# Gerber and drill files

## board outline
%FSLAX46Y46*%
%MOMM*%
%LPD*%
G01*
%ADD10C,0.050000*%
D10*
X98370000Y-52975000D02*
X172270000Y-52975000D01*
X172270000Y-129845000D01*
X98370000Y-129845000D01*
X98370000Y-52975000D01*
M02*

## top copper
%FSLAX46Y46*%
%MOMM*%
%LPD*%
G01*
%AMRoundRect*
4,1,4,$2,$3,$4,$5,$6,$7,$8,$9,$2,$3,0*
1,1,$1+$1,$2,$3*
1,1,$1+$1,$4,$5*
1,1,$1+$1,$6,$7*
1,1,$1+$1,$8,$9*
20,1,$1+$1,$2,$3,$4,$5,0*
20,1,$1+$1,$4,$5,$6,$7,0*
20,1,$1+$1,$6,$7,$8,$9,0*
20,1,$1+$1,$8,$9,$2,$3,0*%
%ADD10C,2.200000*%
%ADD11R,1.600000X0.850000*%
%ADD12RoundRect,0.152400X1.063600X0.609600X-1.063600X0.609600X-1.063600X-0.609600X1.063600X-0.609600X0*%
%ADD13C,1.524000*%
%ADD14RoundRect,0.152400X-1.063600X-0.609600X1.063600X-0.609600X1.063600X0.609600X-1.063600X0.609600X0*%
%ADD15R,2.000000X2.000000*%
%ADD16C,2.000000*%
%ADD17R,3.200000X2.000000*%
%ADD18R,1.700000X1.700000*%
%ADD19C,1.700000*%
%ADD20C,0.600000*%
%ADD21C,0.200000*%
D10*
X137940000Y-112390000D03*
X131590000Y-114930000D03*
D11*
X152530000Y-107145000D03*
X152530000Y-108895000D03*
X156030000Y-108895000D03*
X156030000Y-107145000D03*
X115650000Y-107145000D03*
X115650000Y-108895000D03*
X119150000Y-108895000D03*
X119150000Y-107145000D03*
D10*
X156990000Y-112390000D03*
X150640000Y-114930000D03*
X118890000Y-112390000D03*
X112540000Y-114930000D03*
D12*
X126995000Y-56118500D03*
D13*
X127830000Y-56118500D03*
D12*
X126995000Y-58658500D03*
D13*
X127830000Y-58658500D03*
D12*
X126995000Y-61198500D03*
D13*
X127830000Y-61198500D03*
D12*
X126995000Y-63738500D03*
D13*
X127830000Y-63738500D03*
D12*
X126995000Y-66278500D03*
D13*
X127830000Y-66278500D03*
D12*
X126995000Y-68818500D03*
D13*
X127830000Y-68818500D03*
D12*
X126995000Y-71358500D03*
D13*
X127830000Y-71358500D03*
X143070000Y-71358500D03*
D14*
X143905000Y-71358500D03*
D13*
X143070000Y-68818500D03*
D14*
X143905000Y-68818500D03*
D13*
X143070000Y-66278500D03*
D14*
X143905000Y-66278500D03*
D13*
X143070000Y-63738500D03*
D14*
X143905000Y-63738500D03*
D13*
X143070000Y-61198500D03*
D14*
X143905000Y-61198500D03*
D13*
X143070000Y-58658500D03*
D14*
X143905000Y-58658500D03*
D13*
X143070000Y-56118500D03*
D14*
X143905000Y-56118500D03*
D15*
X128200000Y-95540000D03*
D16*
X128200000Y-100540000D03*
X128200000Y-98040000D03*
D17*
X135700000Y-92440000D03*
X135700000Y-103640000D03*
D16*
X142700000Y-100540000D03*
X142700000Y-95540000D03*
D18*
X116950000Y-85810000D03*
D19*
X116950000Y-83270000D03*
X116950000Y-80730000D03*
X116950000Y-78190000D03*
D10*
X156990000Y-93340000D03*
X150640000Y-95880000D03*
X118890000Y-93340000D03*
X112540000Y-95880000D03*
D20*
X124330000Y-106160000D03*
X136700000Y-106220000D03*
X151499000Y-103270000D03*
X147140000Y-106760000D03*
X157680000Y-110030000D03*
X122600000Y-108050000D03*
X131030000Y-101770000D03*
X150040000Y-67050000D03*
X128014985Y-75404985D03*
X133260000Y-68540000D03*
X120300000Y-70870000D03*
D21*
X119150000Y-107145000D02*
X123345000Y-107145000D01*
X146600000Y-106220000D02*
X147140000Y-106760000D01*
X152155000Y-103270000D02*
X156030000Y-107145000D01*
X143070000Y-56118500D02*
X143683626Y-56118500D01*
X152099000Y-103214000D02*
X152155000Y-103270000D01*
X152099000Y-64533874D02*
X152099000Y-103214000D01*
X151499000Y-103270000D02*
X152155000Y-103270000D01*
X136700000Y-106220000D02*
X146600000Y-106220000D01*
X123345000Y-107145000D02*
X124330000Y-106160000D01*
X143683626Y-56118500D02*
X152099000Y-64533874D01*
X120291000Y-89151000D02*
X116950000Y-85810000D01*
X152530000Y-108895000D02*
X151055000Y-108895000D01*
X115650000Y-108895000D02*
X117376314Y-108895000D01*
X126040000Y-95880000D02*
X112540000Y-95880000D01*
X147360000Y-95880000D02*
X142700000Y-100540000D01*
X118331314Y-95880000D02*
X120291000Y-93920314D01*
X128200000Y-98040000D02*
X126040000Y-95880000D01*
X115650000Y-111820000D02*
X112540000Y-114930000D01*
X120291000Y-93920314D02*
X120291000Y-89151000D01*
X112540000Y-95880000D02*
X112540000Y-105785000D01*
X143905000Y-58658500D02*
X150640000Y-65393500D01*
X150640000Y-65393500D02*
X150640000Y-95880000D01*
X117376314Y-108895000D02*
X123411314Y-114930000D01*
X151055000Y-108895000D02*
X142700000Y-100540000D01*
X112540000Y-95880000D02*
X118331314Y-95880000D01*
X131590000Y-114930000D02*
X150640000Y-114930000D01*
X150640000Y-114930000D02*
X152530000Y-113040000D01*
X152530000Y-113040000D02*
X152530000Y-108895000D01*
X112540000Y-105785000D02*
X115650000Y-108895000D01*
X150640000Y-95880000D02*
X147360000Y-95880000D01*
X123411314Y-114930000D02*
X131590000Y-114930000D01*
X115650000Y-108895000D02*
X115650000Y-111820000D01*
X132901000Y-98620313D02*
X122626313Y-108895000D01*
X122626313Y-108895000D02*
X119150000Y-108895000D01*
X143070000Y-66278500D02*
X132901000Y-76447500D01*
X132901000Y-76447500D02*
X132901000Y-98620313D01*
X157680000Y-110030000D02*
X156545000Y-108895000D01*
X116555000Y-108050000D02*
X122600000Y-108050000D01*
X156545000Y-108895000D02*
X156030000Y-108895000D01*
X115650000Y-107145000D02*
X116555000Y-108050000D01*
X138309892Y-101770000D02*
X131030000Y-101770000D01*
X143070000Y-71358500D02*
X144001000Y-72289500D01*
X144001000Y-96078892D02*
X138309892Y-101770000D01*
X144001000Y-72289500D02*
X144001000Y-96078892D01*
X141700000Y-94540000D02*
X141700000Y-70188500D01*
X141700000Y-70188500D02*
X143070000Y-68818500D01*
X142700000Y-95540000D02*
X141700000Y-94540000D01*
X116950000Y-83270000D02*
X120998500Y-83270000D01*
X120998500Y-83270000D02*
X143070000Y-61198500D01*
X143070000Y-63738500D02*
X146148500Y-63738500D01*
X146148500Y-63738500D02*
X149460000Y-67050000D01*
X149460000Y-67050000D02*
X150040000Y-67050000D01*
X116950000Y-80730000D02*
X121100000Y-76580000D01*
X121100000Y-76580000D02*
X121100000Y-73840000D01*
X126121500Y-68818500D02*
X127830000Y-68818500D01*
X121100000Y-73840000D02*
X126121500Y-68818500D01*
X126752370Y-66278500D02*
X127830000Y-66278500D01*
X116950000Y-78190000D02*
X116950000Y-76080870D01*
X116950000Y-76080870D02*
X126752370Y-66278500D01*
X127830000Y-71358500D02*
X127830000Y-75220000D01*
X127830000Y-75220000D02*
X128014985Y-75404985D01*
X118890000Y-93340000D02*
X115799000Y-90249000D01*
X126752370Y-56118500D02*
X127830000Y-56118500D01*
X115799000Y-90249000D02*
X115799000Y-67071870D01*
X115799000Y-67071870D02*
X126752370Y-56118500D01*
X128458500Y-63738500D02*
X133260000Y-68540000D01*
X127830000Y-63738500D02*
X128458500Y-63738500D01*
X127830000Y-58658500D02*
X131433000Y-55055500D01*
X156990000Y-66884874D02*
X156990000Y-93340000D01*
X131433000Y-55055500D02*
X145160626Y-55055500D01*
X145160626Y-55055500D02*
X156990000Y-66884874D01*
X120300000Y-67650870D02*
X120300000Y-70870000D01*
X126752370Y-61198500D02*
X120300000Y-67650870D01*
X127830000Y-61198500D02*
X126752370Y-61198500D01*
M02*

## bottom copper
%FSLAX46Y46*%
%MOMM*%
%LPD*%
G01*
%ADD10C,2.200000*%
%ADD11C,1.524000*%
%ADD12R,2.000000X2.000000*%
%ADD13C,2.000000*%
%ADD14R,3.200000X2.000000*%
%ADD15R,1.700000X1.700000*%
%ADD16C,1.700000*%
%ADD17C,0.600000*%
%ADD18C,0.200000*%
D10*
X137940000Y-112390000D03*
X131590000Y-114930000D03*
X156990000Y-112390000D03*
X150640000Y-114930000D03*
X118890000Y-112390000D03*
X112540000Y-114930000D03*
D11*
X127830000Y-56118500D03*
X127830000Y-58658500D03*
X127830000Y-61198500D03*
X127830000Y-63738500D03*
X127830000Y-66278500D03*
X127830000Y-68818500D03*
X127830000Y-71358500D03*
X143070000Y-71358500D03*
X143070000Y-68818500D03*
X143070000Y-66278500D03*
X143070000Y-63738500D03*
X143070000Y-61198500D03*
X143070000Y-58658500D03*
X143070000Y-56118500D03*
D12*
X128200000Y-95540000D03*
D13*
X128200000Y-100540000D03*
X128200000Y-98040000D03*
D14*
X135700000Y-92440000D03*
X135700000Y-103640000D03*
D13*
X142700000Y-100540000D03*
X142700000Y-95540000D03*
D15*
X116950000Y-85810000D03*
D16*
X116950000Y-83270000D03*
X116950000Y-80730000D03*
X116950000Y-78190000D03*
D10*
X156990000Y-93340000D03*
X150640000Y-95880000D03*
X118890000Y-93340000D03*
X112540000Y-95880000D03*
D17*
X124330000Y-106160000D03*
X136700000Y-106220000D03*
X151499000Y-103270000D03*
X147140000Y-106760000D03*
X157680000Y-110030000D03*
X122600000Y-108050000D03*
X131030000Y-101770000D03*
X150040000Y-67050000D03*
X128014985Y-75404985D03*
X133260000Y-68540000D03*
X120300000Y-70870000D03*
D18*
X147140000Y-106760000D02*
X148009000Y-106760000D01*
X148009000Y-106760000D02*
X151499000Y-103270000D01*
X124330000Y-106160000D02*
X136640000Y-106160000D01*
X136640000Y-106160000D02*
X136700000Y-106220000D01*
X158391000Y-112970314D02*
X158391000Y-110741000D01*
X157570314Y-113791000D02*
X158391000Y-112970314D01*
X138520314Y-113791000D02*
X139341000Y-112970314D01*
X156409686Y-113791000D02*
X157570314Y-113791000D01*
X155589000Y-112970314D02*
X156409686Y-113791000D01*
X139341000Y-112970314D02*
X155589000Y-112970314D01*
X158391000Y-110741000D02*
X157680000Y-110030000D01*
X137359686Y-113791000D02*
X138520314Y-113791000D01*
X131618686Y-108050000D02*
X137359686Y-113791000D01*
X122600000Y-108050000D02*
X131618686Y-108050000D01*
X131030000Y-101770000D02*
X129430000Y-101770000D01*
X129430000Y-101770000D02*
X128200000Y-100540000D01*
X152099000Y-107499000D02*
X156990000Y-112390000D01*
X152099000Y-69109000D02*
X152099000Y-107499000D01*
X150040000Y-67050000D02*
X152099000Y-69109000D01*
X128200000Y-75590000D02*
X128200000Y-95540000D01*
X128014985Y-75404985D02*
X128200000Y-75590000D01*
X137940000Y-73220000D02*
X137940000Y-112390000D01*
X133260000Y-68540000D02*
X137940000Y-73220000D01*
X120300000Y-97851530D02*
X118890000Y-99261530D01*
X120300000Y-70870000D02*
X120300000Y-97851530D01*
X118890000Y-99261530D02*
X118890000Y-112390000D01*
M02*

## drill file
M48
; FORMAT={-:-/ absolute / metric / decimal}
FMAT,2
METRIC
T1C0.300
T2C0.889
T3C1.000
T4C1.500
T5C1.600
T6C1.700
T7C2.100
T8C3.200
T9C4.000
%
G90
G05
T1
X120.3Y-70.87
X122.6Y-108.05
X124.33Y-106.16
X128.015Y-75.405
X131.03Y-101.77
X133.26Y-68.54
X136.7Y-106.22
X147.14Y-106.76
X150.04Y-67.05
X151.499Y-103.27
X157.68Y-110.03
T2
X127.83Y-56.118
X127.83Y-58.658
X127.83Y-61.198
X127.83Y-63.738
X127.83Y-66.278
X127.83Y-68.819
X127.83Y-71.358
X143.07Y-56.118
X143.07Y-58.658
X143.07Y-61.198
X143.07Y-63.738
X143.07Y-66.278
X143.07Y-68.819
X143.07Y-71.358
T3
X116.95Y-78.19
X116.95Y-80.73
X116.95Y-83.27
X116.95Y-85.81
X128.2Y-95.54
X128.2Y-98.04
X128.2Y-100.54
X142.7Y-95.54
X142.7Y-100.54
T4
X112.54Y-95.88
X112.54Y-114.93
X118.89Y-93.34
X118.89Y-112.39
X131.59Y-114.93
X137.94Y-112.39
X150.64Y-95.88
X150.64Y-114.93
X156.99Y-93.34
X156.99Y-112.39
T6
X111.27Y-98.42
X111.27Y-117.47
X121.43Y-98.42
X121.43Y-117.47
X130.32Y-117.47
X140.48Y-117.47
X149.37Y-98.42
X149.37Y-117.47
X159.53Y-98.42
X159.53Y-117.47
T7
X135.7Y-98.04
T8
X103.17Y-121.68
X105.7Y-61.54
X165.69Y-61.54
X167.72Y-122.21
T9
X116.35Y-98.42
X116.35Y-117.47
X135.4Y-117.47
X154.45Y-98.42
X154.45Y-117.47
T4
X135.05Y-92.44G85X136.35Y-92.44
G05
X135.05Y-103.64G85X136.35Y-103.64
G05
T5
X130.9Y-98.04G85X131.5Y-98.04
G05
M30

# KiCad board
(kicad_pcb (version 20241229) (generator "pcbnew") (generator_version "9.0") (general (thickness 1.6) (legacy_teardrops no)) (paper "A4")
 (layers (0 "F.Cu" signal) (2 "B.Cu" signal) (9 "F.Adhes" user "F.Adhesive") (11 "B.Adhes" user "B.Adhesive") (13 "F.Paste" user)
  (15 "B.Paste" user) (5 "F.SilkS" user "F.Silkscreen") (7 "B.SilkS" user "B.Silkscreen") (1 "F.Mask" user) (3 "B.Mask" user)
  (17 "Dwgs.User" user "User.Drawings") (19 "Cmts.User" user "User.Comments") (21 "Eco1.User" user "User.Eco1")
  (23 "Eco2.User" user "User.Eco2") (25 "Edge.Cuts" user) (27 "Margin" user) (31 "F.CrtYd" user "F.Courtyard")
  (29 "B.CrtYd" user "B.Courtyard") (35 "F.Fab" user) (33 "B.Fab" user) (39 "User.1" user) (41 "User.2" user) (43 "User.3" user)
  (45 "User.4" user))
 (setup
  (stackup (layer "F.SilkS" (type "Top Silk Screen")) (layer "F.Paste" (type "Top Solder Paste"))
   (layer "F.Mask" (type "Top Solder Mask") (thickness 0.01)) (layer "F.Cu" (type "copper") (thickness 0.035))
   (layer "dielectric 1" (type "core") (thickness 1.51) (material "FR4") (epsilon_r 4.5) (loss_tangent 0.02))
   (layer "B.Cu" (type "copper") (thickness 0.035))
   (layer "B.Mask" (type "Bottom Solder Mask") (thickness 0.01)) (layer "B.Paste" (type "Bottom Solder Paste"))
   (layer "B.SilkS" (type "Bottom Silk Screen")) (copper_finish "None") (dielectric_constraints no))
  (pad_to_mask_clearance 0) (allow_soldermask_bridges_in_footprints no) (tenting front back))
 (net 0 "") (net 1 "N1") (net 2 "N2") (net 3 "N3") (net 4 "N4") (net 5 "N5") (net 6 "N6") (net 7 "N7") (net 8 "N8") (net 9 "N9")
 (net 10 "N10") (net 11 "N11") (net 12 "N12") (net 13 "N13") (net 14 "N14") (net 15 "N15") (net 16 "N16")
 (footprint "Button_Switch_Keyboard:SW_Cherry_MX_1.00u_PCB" (layer "F.Cu") (at 137.94 112.39)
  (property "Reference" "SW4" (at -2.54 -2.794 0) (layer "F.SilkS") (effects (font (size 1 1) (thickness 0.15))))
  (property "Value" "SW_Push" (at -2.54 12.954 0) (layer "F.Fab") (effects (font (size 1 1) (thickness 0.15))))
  (pad "" np_thru_hole circle (at -7.62 5.08) (size 1.7 1.7) (drill 1.7) (layers "*.Cu" "*.Mask"))
  (pad "" np_thru_hole circle (at -2.54 5.08) (size 4 4) (drill 4) (layers "*.Cu" "*.Mask"))
  (pad "" np_thru_hole circle (at 2.54 5.08) (size 1.7 1.7) (drill 1.7) (layers "*.Cu" "*.Mask"))
  (pad "1" thru_hole circle (at 0 0) (size 2.2 2.2) (drill 1.5) (layers "*.Cu" "*.Mask") (remove_unused_layers no) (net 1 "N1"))
  (pad "2" thru_hole circle (at -6.35 2.54) (size 2.2 2.2) (drill 1.5) (layers "*.Cu" "*.Mask") (remove_unused_layers no) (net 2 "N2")))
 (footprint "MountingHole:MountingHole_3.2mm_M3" (layer "F.Cu") (at 105.7 61.54 -90)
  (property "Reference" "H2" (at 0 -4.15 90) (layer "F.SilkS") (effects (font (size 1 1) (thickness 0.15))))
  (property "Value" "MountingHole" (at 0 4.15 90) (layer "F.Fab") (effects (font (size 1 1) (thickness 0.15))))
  (pad "" np_thru_hole circle (at 0 0 270) (size 3.2 3.2) (drill 3.2) (layers "*.Cu" "*.Mask")))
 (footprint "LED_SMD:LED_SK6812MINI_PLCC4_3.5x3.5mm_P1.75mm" (layer "F.Cu") (at 154.28 108.02)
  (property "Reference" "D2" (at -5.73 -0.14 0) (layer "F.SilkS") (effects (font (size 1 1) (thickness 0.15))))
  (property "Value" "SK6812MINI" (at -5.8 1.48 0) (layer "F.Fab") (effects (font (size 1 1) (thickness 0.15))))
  (pad "1" smd rect (at -1.75 -0.875) (size 1.6 0.85) (layers "F.Cu" "F.Mask" "F.Paste") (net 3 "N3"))
  (pad "2" smd rect (at -1.75 0.875) (size 1.6 0.85) (layers "F.Cu" "F.Mask" "F.Paste") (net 2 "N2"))
  (pad "3" smd rect (at 1.75 0.875) (size 1.6 0.85) (layers "F.Cu" "F.Mask" "F.Paste") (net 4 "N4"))
  (pad "4" smd rect (at 1.75 -0.875) (size 1.6 0.85) (layers "F.Cu" "F.Mask" "F.Paste") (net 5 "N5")))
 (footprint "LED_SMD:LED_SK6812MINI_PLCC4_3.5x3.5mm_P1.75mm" (layer "F.Cu") (at 117.4 108.02)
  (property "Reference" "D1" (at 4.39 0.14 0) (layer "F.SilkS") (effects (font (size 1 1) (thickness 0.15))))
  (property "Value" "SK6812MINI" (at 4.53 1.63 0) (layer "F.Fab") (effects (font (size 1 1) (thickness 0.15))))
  (pad "1" smd rect (at -1.75 -0.875) (size 1.6 0.85) (layers "F.Cu" "F.Mask" "F.Paste") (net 4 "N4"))
  (pad "2" smd rect (at -1.75 0.875) (size 1.6 0.85) (layers "F.Cu" "F.Mask" "F.Paste") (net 2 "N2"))
  (pad "3" smd rect (at 1.75 0.875) (size 1.6 0.85) (layers "F.Cu" "F.Mask" "F.Paste") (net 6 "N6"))
  (pad "4" smd rect (at 1.75 -0.875) (size 1.6 0.85) (layers "F.Cu" "F.Mask" "F.Paste") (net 5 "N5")))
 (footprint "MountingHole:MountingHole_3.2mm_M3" (layer "F.Cu") (at 165.69 61.54 90)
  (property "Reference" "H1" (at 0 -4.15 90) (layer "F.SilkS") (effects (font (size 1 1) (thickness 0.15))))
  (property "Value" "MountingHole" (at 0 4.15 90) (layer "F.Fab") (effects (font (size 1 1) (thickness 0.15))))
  (pad "" np_thru_hole circle (at 0 0 90) (size 3.2 3.2) (drill 3.2) (layers "*.Cu" "*.Mask")))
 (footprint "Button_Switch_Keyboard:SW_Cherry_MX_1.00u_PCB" (layer "F.Cu") (at 156.99 112.39)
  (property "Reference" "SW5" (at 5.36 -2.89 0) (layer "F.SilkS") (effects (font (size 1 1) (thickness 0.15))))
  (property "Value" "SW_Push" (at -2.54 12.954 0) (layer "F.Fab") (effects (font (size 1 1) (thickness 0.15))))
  (pad "" np_thru_hole circle (at -7.62 5.08) (size 1.7 1.7) (drill 1.7) (layers "*.Cu" "*.Mask"))
  (pad "" np_thru_hole circle (at -2.54 5.08) (size 4 4) (drill 4) (layers "*.Cu" "*.Mask"))
  (pad "" np_thru_hole circle (at 2.54 5.08) (size 1.7 1.7) (drill 1.7) (layers "*.Cu" "*.Mask"))
  (pad "1" thru_hole circle (at 0 0) (size 2.2 2.2) (drill 1.5) (layers "*.Cu" "*.Mask") (remove_unused_layers no) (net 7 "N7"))
  (pad "2" thru_hole circle (at -6.35 2.54) (size 2.2 2.2) (drill 1.5) (layers "*.Cu" "*.Mask") (remove_unused_layers no) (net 2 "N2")))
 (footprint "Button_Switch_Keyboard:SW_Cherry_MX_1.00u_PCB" (layer "F.Cu") (at 118.89 112.39)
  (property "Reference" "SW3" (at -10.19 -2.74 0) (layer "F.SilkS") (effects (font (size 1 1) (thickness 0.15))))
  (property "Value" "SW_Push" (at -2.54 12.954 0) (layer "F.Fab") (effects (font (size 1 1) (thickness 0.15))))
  (pad "" np_thru_hole circle (at -7.62 5.08) (size 1.7 1.7) (drill 1.7) (layers "*.Cu" "*.Mask"))
  (pad "" np_thru_hole circle (at -2.54 5.08) (size 4 4) (drill 4) (layers "*.Cu" "*.Mask"))
  (pad "" np_thru_hole circle (at 2.54 5.08) (size 1.7 1.7) (drill 1.7) (layers "*.Cu" "*.Mask"))
  (pad "1" thru_hole circle (at 0 0) (size 2.2 2.2) (drill 1.5) (layers "*.Cu" "*.Mask") (remove_unused_layers no) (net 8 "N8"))
  (pad "2" thru_hole circle (at -6.35 2.54) (size 2.2 2.2) (drill 1.5) (layers "*.Cu" "*.Mask") (remove_unused_layers no) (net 2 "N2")))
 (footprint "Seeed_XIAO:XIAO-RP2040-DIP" (layer "F.Cu") (at 135.45 63.7385)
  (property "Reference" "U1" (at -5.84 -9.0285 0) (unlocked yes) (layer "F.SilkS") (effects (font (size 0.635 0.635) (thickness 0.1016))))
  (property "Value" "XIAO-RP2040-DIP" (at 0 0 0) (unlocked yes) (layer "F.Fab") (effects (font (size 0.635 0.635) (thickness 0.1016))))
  (pad "1" smd roundrect (at -8.455 -7.62 180) (size 2.432 1.524) (layers "F.Cu" "F.Mask") (roundrect_rratio 0.1) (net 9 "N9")
   (thermal_bridge_angle 45))
  (pad "1" thru_hole circle (at -7.62 -7.62 180) (size 1.524 1.524) (drill 0.889) (layers "*.Cu" "*.Mask") (remove_unused_layers no)
   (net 9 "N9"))
  (pad "2" smd roundrect (at -8.455 -5.08 180) (size 2.432 1.524) (layers "F.Cu" "F.Mask") (roundrect_rratio 0.1) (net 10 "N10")
   (thermal_bridge_angle 45))
  (pad "2" thru_hole circle (at -7.62 -5.08 180) (size 1.524 1.524) (drill 0.889) (layers "*.Cu" "*.Mask") (remove_unused_layers no)
   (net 10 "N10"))
  (pad "3" smd roundrect (at -8.455 -2.54 180) (size 2.432 1.524) (layers "F.Cu" "F.Mask") (roundrect_rratio 0.1) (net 8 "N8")
   (thermal_bridge_angle 45))
  (pad "3" thru_hole circle (at -7.62 -2.54 180) (size 1.524 1.524) (drill 0.889) (layers "*.Cu" "*.Mask") (remove_unused_layers no)
   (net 8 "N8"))
  (pad "4" smd roundrect (at -8.455 0 180) (size 2.432 1.524) (layers "F.Cu" "F.Mask") (roundrect_rratio 0.1) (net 1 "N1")
   (thermal_bridge_angle 45))
  (pad "4" thru_hole circle (at -7.62 0 180) (size 1.524 1.524) (drill 0.889) (layers "*.Cu" "*.Mask") (remove_unused_layers no)
   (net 1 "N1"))
  (pad "5" smd roundrect (at -8.455 2.54 180) (size 2.432 1.524) (layers "F.Cu" "F.Mask") (roundrect_rratio 0.1) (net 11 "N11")
   (thermal_bridge_angle 45))
  (pad "5" thru_hole circle (at -7.62 2.54 180) (size 1.524 1.524) (drill 0.889) (layers "*.Cu" "*.Mask") (remove_unused_layers no)
   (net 11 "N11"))
  (pad "6" smd roundrect (at -8.455 5.08 180) (size 2.432 1.524) (layers "F.Cu" "F.Mask") (roundrect_rratio 0.1) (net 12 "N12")
   (thermal_bridge_angle 45))
  (pad "6" thru_hole circle (at -7.62 5.08 180) (size 1.524 1.524) (drill 0.889) (layers "*.Cu" "*.Mask") (remove_unused_layers no)
   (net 12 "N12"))
  (pad "7" smd roundrect (at -8.455 7.62 180) (size 2.432 1.524) (layers "F.Cu" "F.Mask") (roundrect_rratio 0.1) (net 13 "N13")
   (thermal_bridge_angle 45))
  (pad "7" thru_hole circle (at -7.62 7.62 180) (size 1.524 1.524) (drill 0.889) (layers "*.Cu" "*.Mask") (remove_unused_layers no)
   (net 13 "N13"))
  (pad "8" thru_hole circle (at 7.62 7.62) (size 1.524 1.524) (drill 0.889) (layers "*.Cu" "*.Mask") (remove_unused_layers no)
   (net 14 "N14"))
  (pad "8" smd roundrect (at 8.455 7.62) (size 2.432 1.524) (layers "F.Cu" "F.Mask") (roundrect_rratio 0.1) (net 14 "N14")
   (thermal_bridge_angle 45))
  (pad "9" thru_hole circle (at 7.62 5.08) (size 1.524 1.524) (drill 0.889) (layers "*.Cu" "*.Mask") (remove_unused_layers no)
   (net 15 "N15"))
  (pad "9" smd roundrect (at 8.455 5.08) (size 2.432 1.524) (layers "F.Cu" "F.Mask") (roundrect_rratio 0.1) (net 15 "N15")
   (thermal_bridge_angle 45))
  (pad "10" thru_hole circle (at 7.62 2.54) (size 1.524 1.524) (drill 0.889) (layers "*.Cu" "*.Mask") (remove_unused_layers no) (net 6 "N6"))
  (pad "10" smd roundrect (at 8.455 2.54) (size 2.432 1.524) (layers "F.Cu" "F.Mask") (roundrect_rratio 0.1) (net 6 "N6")
   (thermal_bridge_angle 45))
  (pad "11" thru_hole circle (at 7.62 0) (size 1.524 1.524) (drill 0.889) (layers "*.Cu" "*.Mask") (remove_unused_layers no) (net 7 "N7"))
  (pad "11" smd roundrect (at 8.455 0) (size 2.432 1.524) (layers "F.Cu" "F.Mask") (roundrect_rratio 0.1) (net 7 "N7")
   (thermal_bridge_angle 45))
  (pad "12" thru_hole circle (at 7.62 -2.54) (size 1.524 1.524) (drill 0.889) (layers "*.Cu" "*.Mask") (remove_unused_layers no)
   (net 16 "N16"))
  (pad "12" smd roundrect (at 8.455 -2.54) (size 2.432 1.524) (layers "F.Cu" "F.Mask") (roundrect_rratio 0.1) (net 16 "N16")
   (thermal_bridge_angle 45))
  (pad "13" thru_hole circle (at 7.62 -5.08) (size 1.524 1.524) (drill 0.889) (layers "*.Cu" "*.Mask") (remove_unused_layers no)
   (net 2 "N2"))
  (pad "13" smd roundrect (at 8.455 -5.08) (size 2.432 1.524) (layers "F.Cu" "F.Mask") (roundrect_rratio 0.1) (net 2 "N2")
   (thermal_bridge_angle 45))
  (pad "14" thru_hole circle (at 7.62 -7.62) (size 1.524 1.524) (drill 0.889) (layers "*.Cu" "*.Mask") (remove_unused_layers no)
   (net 5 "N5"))
  (pad "14" smd roundrect (at 8.455 -7.62) (size 2.432 1.524) (layers "F.Cu" "F.Mask") (roundrect_rratio 0.1) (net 5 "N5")
   (thermal_bridge_angle 45)))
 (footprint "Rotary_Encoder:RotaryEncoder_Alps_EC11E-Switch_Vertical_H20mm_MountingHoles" (layer "F.Cu") (at 128.2 95.54)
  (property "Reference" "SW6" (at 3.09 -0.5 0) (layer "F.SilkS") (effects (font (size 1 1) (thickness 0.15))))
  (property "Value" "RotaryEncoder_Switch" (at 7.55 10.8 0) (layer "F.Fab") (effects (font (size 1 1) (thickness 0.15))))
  (pad "" np_thru_hole oval (at 3 2.5) (size 2.2 1.6) (drill oval 2.2 1.6) (layers "*.Mask"))
  (pad "" np_thru_hole circle (at 7.5 2.5) (size 2.1 2.1) (drill 2.1) (layers "*.Mask"))
  (pad "A" thru_hole rect (at 0 0) (size 2 2) (drill 1) (layers "*.Cu" "*.Mask") (remove_unused_layers no) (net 13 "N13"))
  (pad "B" thru_hole circle (at 0 5) (size 2 2) (drill 1) (layers "*.Cu" "*.Mask") (remove_unused_layers no) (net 14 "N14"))
  (pad "C" thru_hole circle (at 0 2.5) (size 2 2) (drill 1) (layers "*.Cu" "*.Mask") (remove_unused_layers no) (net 2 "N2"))
  (pad "MP" thru_hole rect (at 7.5 -3.1) (size 3.2 2) (drill oval 2.8 1.5) (layers "*.Cu" "*.Mask") (remove_unused_layers no))
  (pad "MP" thru_hole rect (at 7.5 8.1) (size 3.2 2) (drill oval 2.8 1.5) (layers "*.Cu" "*.Mask") (remove_unused_layers no))
  (pad "S1" thru_hole circle (at 14.5 5) (size 2 2) (drill 1) (layers "*.Cu" "*.Mask") (remove_unused_layers no) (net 2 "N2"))
  (pad "S2" thru_hole circle (at 14.5 0) (size 2 2) (drill 1) (layers "*.Cu" "*.Mask") (remove_unused_layers no) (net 15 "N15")))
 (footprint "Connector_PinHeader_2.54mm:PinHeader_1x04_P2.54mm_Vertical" (layer "F.Cu") (at 116.95 85.81 180)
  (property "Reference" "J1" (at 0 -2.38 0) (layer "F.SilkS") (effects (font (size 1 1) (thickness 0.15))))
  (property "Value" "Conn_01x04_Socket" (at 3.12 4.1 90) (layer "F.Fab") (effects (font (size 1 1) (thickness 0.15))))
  (pad "1" thru_hole rect (at 0 0 180) (size 1.7 1.7) (drill 1) (layers "*.Cu" "*.Mask") (remove_unused_layers no) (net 2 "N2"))
  (pad "2" thru_hole circle (at 0 2.54 180) (size 1.7 1.7) (drill 1) (layers "*.Cu" "*.Mask") (remove_unused_layers no) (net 16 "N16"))
  (pad "3" thru_hole circle (at 0 5.08 180) (size 1.7 1.7) (drill 1) (layers "*.Cu" "*.Mask") (remove_unused_layers no) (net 12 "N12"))
  (pad "4" thru_hole circle (at 0 7.62 180) (size 1.7 1.7) (drill 1) (layers "*.Cu" "*.Mask") (remove_unused_layers no) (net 11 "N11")))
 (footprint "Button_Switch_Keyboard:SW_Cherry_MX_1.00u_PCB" (layer "F.Cu") (at 156.99 93.34)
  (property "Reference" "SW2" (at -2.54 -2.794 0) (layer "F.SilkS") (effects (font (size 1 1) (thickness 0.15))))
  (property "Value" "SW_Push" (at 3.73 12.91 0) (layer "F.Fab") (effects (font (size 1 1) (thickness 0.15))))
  (pad "" np_thru_hole circle (at -7.62 5.08) (size 1.7 1.7) (drill 1.7) (layers "*.Cu" "*.Mask"))
  (pad "" np_thru_hole circle (at -2.54 5.08) (size 4 4) (drill 4) (layers "*.Cu" "*.Mask"))
  (pad "" np_thru_hole circle (at 2.54 5.08) (size 1.7 1.7) (drill 1.7) (layers "*.Cu" "*.Mask"))
  (pad "1" thru_hole circle (at 0 0) (size 2.2 2.2) (drill 1.5) (layers "*.Cu" "*.Mask") (remove_unused_layers no) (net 10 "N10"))
  (pad "2" thru_hole circle (at -6.35 2.54) (size 2.2 2.2) (drill 1.5) (layers "*.Cu" "*.Mask") (remove_unused_layers no) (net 2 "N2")))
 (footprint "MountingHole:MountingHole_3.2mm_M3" (layer "F.Cu") (at 103.17 121.68 180)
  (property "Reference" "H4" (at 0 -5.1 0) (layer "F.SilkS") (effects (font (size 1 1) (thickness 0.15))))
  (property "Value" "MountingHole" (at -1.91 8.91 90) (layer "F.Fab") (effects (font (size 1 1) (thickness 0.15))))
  (pad "" np_thru_hole circle (at 0 0 180) (size 3.2 3.2) (drill 3.2) (layers "*.Cu" "*.Mask")))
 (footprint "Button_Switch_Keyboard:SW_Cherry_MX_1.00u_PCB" (layer "F.Cu") (at 118.89 93.34)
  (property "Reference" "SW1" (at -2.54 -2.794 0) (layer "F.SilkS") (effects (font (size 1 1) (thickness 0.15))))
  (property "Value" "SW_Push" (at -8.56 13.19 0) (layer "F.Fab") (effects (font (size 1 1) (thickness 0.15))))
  (pad "" np_thru_hole circle (at -7.62 5.08) (size 1.7 1.7) (drill 1.7) (layers "*.Cu" "*.Mask"))
  (pad "" np_thru_hole circle (at -2.54 5.08) (size 4 4) (drill 4) (layers "*.Cu" "*.Mask"))
  (pad "" np_thru_hole circle (at 2.54 5.08) (size 1.7 1.7) (drill 1.7) (layers "*.Cu" "*.Mask"))
  (pad "1" thru_hole circle (at 0 0) (size 2.2 2.2) (drill 1.5) (layers "*.Cu" "*.Mask") (remove_unused_layers no) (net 9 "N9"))
  (pad "2" thru_hole circle (at -6.35 2.54) (size 2.2 2.2) (drill 1.5) (layers "*.Cu" "*.Mask") (remove_unused_layers no) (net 2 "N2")))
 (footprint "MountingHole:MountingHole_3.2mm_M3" (layer "F.Cu") (at 167.72 122.21 180)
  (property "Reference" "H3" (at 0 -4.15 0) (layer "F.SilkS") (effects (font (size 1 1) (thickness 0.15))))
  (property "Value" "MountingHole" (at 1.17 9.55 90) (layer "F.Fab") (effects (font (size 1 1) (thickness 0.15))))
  (pad "" np_thru_hole circle (at 0 0 180) (size 3.2 3.2) (drill 3.2) (layers "*.Cu" "*.Mask")))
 (gr_rect (start 98.37 52.975) (end 172.27 129.845) (stroke (width 0.05) (type solid)) (fill no) (layer "Edge.Cuts"))
 (segment (start 119.15 107.145) (end 123.345 107.145) (width 0.2) (layer "F.Cu") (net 5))
 (segment (start 146.6 106.22) (end 147.14 106.76) (width 0.2) (layer "F.Cu") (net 5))
 (segment (start 152.155 103.27) (end 156.03 107.145) (width 0.2) (layer "F.Cu") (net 5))
 (segment (start 143.07 56.1185) (end 143.683626 56.1185) (width 0.2) (layer "F.Cu") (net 5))
 (segment (start 152.099 103.214) (end 152.155 103.27) (width 0.2) (layer "F.Cu") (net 5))
 (segment (start 152.099 64.533874) (end 152.099 103.214) (width 0.2) (layer "F.Cu") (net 5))
 (segment (start 151.499 103.27) (end 152.155 103.27) (width 0.2) (layer "F.Cu") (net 5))
 (segment (start 136.7 106.22) (end 146.6 106.22) (width 0.2) (layer "F.Cu") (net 5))
 (segment (start 123.345 107.145) (end 124.33 106.16) (width 0.2) (layer "F.Cu") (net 5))
 (segment (start 143.683626 56.1185) (end 152.099 64.533874) (width 0.2) (layer "F.Cu") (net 5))
 (via (at 124.33 106.16) (size 0.6) (drill 0.3) (layers "F.Cu" "B.Cu") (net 5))
 (via (at 136.7 106.22) (size 0.6) (drill 0.3) (layers "F.Cu" "B.Cu") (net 5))
 (via (at 151.499 103.27) (size 0.6) (drill 0.3) (layers "F.Cu" "B.Cu") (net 5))
 (via (at 147.14 106.76) (size 0.6) (drill 0.3) (layers "F.Cu" "B.Cu") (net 5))
 (segment (start 147.14 106.76) (end 148.009 106.76) (width 0.2) (layer "B.Cu") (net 5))
 (segment (start 148.009 106.76) (end 151.499 103.27) (width 0.2) (layer "B.Cu") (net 5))
 (segment (start 124.33 106.16) (end 136.64 106.16) (width 0.2) (layer "B.Cu") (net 5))
 (segment (start 136.64 106.16) (end 136.7 106.22) (width 0.2) (layer "B.Cu") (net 5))
 (segment (start 120.291 89.151) (end 116.95 85.81) (width 0.2) (layer "F.Cu") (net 2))
 (segment (start 152.53 108.895) (end 151.055 108.895) (width 0.2) (layer "F.Cu") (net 2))
 (segment (start 115.65 108.895) (end 117.376314 108.895) (width 0.2) (layer "F.Cu") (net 2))
 (segment (start 126.04 95.88) (end 112.54 95.88) (width 0.2) (layer "F.Cu") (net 2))
 (segment (start 147.36 95.88) (end 142.7 100.54) (width 0.2) (layer "F.Cu") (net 2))
 (segment (start 118.331314 95.88) (end 120.291 93.920314) (width 0.2) (layer "F.Cu") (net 2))
 (segment (start 128.2 98.04) (end 126.04 95.88) (width 0.2) (layer "F.Cu") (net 2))
 (segment (start 115.65 111.82) (end 112.54 114.93) (width 0.2) (layer "F.Cu") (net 2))
 (segment (start 120.291 93.920314) (end 120.291 89.151) (width 0.2) (layer "F.Cu") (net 2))
 (segment (start 112.54 95.88) (end 112.54 105.785) (width 0.2) (layer "F.Cu") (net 2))
 (segment (start 143.905 58.6585) (end 150.64 65.3935) (width 0.2) (layer "F.Cu") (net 2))
 (segment (start 150.64 65.3935) (end 150.64 95.88) (width 0.2) (layer "F.Cu") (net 2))
 (segment (start 117.376314 108.895) (end 123.411314 114.93) (width 0.2) (layer "F.Cu") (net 2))
 (segment (start 151.055 108.895) (end 142.7 100.54) (width 0.2) (layer "F.Cu") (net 2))
 (segment (start 112.54 95.88) (end 118.331314 95.88) (width 0.2) (layer "F.Cu") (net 2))
 (segment (start 131.59 114.93) (end 150.64 114.93) (width 0.2) (layer "F.Cu") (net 2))
 (segment (start 150.64 114.93) (end 152.53 113.04) (width 0.2) (layer "F.Cu") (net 2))
 (segment (start 152.53 113.04) (end 152.53 108.895) (width 0.2) (layer "F.Cu") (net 2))
 (segment (start 112.54 105.785) (end 115.65 108.895) (width 0.2) (layer "F.Cu") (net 2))
 (segment (start 150.64 95.88) (end 147.36 95.88) (width 0.2) (layer "F.Cu") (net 2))
 (segment (start 123.411314 114.93) (end 131.59 114.93) (width 0.2) (layer "F.Cu") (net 2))
 (segment (start 115.65 108.895) (end 115.65 111.82) (width 0.2) (layer "F.Cu") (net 2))
 (segment (start 132.901 98.620313) (end 122.626313 108.895) (width 0.2) (layer "F.Cu") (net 6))
 (segment (start 122.626313 108.895) (end 119.15 108.895) (width 0.2) (layer "F.Cu") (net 6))
 (segment (start 143.07 66.2785) (end 132.901 76.4475) (width 0.2) (layer "F.Cu") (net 6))
 (segment (start 132.901 76.4475) (end 132.901 98.620313) (width 0.2) (layer "F.Cu") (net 6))
 (segment (start 157.68 110.03) (end 156.545 108.895) (width 0.2) (layer "F.Cu") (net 4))
 (segment (start 116.555 108.05) (end 122.6 108.05) (width 0.2) (layer "F.Cu") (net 4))
 (segment (start 156.545 108.895) (end 156.03 108.895) (width 0.2) (layer "F.Cu") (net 4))
 (segment (start 115.65 107.145) (end 116.555 108.05) (width 0.2) (layer "F.Cu") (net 4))
 (via (at 157.68 110.03) (size 0.6) (drill 0.3) (layers "F.Cu" "B.Cu") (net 4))
 (via (at 122.6 108.05) (size 0.6) (drill 0.3) (layers "F.Cu" "B.Cu") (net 4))
 (segment (start 158.391 112.970314) (end 158.391 110.741) (width 0.2) (layer "B.Cu") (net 4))
 (segment (start 157.570314 113.791) (end 158.391 112.970314) (width 0.2) (layer "B.Cu") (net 4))
 (segment (start 138.520314 113.791) (end 139.341 112.970314) (width 0.2) (layer "B.Cu") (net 4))
 (segment (start 156.409686 113.791) (end 157.570314 113.791) (width 0.2) (layer "B.Cu") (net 4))
 (segment (start 155.589 112.970314) (end 156.409686 113.791) (width 0.2) (layer "B.Cu") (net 4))
 (segment (start 139.341 112.970314) (end 155.589 112.970314) (width 0.2) (layer "B.Cu") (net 4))
 (segment (start 158.391 110.741) (end 157.68 110.03) (width 0.2) (layer "B.Cu") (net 4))
 (segment (start 137.359686 113.791) (end 138.520314 113.791) (width 0.2) (layer "B.Cu") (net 4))
 (segment (start 131.618686 108.05) (end 137.359686 113.791) (width 0.2) (layer "B.Cu") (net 4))
 (segment (start 122.6 108.05) (end 131.618686 108.05) (width 0.2) (layer "B.Cu") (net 4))
 (segment (start 138.309892 101.77) (end 131.03 101.77) (width 0.2) (layer "F.Cu") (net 14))
 (segment (start 143.07 71.3585) (end 144.001 72.2895) (width 0.2) (layer "F.Cu") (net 14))
 (segment (start 144.001 96.078892) (end 138.309892 101.77) (width 0.2) (layer "F.Cu") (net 14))
 (segment (start 144.001 72.2895) (end 144.001 96.078892) (width 0.2) (layer "F.Cu") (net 14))
 (via (at 131.03 101.77) (size 0.6) (drill 0.3) (layers "F.Cu" "B.Cu") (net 14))
 (segment (start 131.03 101.77) (end 129.43 101.77) (width 0.2) (layer "B.Cu") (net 14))
 (segment (start 129.43 101.77) (end 128.2 100.54) (width 0.2) (layer "B.Cu") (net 14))
 (segment (start 141.7 94.54) (end 141.7 70.1885) (width 0.2) (layer "F.Cu") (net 15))
 (segment (start 141.7 70.1885) (end 143.07 68.8185) (width 0.2) (layer "F.Cu") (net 15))
 (segment (start 142.7 95.54) (end 141.7 94.54) (width 0.2) (layer "F.Cu") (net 15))
 (segment (start 116.95 83.27) (end 120.9985 83.27) (width 0.2) (layer "F.Cu") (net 16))
 (segment (start 120.9985 83.27) (end 143.07 61.1985) (width 0.2) (layer "F.Cu") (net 16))
 (segment (start 143.07 63.7385) (end 146.1485 63.7385) (width 0.2) (layer "F.Cu") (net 7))
 (segment (start 146.1485 63.7385) (end 149.46 67.05) (width 0.2) (layer "F.Cu") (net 7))
 (segment (start 149.46 67.05) (end 150.04 67.05) (width 0.2) (layer "F.Cu") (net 7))
 (via (at 150.04 67.05) (size 0.6) (drill 0.3) (layers "F.Cu" "B.Cu") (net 7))
 (segment (start 152.099 107.499) (end 156.99 112.39) (width 0.2) (layer "B.Cu") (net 7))
 (segment (start 152.099 69.109) (end 152.099 107.499) (width 0.2) (layer "B.Cu") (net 7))
 (segment (start 150.04 67.05) (end 152.099 69.109) (width 0.2) (layer "B.Cu") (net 7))
 (segment (start 116.95 80.73) (end 121.1 76.58) (width 0.2) (layer "F.Cu") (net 12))
 (segment (start 121.1 76.58) (end 121.1 73.84) (width 0.2) (layer "F.Cu") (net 12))
 (segment (start 126.1215 68.8185) (end 127.83 68.8185) (width 0.2) (layer "F.Cu") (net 12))
 (segment (start 121.1 73.84) (end 126.1215 68.8185) (width 0.2) (layer "F.Cu") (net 12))
 (segment (start 126.75237 66.2785) (end 127.83 66.2785) (width 0.2) (layer "F.Cu") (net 11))
 (segment (start 116.95 78.19) (end 116.95 76.08087) (width 0.2) (layer "F.Cu") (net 11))
 (segment (start 116.95 76.08087) (end 126.75237 66.2785) (width 0.2) (layer "F.Cu") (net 11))
 (segment (start 127.83 71.3585) (end 127.83 75.22) (width 0.2) (layer "F.Cu") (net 13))
 (segment (start 127.83 75.22) (end 128.014985 75.404985) (width 0.2) (layer "F.Cu") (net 13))
 (via (at 128.014985 75.404985) (size 0.6) (drill 0.3) (layers "F.Cu" "B.Cu") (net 13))
 (segment (start 128.2 75.59) (end 128.2 95.54) (width 0.2) (layer "B.Cu") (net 13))
 (segment (start 128.014985 75.404985) (end 128.2 75.59) (width 0.2) (layer "B.Cu") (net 13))
 (segment (start 118.89 93.34) (end 115.799 90.249) (width 0.2) (layer "F.Cu") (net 9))
 (segment (start 126.75237 56.1185) (end 127.83 56.1185) (width 0.2) (layer "F.Cu") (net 9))
 (segment (start 115.799 90.249) (end 115.799 67.07187) (width 0.2) (layer "F.Cu") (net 9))
 (segment (start 115.799 67.07187) (end 126.75237 56.1185) (width 0.2) (layer "F.Cu") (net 9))
 (segment (start 128.4585 63.7385) (end 133.26 68.54) (width 0.2) (layer "F.Cu") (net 1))
 (segment (start 127.83 63.7385) (end 128.4585 63.7385) (width 0.2) (layer "F.Cu") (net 1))
 (via (at 133.26 68.54) (size 0.6) (drill 0.3) (layers "F.Cu" "B.Cu") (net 1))
 (segment (start 137.94 73.22) (end 137.94 112.39) (width 0.2) (layer "B.Cu") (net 1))
 (segment (start 133.26 68.54) (end 137.94 73.22) (width 0.2) (layer "B.Cu") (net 1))
 (segment (start 127.83 58.6585) (end 131.433 55.0555) (width 0.2) (layer "F.Cu") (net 10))
 (segment (start 156.99 66.884874) (end 156.99 93.34) (width 0.2) (layer "F.Cu") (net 10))
 (segment (start 131.433 55.0555) (end 145.160626 55.0555) (width 0.2) (layer "F.Cu") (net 10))
 (segment (start 145.160626 55.0555) (end 156.99 66.884874) (width 0.2) (layer "F.Cu") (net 10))
 (segment (start 120.3 67.65087) (end 120.3 70.87) (width 0.2) (layer "F.Cu") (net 8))
 (segment (start 126.75237 61.1985) (end 120.3 67.65087) (width 0.2) (layer "F.Cu") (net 8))
 (segment (start 127.83 61.1985) (end 126.75237 61.1985) (width 0.2) (layer "F.Cu") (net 8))
 (via (at 120.3 70.87) (size 0.6) (drill 0.3) (layers "F.Cu" "B.Cu") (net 8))
 (segment (start 120.3 97.85153) (end 118.89 99.26153) (width 0.2) (layer "B.Cu") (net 8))
 (segment (start 120.3 70.87) (end 120.3 97.85153) (width 0.2) (layer "B.Cu") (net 8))
 (segment (start 118.89 99.26153) (end 118.89 112.39) (width 0.2) (layer "B.Cu") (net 8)))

